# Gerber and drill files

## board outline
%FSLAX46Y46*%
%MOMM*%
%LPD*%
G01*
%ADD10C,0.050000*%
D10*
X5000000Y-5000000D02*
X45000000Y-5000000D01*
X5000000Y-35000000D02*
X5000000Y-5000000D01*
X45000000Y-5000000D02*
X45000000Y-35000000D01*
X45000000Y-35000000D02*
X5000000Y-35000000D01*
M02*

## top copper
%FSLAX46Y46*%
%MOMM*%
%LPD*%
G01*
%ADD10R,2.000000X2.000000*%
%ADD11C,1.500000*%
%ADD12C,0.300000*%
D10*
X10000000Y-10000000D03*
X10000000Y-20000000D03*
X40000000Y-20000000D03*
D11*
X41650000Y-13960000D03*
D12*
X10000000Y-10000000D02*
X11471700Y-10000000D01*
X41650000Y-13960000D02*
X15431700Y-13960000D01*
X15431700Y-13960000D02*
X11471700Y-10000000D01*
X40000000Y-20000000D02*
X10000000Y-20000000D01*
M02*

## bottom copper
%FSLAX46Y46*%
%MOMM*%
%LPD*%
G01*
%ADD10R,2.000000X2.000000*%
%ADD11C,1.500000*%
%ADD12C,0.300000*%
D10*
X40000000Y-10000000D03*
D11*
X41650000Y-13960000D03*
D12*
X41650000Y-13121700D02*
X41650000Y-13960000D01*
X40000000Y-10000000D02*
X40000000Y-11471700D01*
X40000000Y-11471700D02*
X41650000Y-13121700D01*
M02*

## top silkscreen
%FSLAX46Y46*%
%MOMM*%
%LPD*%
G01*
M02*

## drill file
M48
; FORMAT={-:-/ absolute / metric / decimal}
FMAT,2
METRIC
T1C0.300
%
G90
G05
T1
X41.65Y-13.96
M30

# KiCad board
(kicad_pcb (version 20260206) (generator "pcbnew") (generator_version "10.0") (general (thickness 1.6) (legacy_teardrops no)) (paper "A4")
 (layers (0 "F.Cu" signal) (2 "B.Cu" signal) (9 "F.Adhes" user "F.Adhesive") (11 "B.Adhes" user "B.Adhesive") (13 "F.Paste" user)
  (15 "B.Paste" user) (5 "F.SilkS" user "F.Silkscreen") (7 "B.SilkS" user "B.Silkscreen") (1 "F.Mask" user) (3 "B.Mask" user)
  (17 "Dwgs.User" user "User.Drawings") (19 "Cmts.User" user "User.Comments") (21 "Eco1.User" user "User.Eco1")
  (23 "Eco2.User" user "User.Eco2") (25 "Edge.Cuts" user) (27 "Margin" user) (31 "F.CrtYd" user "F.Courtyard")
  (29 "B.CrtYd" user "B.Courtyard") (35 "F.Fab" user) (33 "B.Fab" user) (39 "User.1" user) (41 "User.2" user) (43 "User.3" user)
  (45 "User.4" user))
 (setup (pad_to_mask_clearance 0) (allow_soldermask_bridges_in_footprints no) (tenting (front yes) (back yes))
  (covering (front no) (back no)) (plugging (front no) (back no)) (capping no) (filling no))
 (gr_line (start 5 5) (end 45 5) (stroke (width 0.05) (type default)) (layer "Edge.Cuts"))
 (gr_line (start 5 35) (end 5 5) (stroke (width 0.05) (type default)) (layer "Edge.Cuts"))
 (gr_line (start 45 5) (end 45 35) (stroke (width 0.05) (type default)) (layer "Edge.Cuts"))
 (gr_line (start 45 35) (end 5 35) (stroke (width 0.05) (type default)) (layer "Edge.Cuts"))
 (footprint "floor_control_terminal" (layer "F.Cu") (at 10 10)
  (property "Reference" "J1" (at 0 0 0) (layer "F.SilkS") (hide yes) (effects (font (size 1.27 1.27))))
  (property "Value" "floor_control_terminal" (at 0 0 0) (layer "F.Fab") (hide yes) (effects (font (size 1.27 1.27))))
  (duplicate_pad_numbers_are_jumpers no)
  (pad "1" smd rect (at 0 0) (size 2 2) (layers "F.Cu" "F.Paste" "F.Mask") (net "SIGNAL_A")))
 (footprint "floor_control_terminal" (layer "B.Cu") (at 40 10)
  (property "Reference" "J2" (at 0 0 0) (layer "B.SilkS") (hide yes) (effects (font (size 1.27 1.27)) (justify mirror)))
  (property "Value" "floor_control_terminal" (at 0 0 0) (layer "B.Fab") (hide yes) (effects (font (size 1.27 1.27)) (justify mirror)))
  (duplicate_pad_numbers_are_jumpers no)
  (pad "1" smd rect (at 0 0) (size 2 2) (layers "B.Cu" "B.Paste" "B.Mask") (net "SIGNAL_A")))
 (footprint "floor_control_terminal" (layer "F.Cu") (at 10 20)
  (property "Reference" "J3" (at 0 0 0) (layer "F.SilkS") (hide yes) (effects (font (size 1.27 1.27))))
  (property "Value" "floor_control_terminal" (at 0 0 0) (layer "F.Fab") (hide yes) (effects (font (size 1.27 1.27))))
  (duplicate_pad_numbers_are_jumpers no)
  (pad "1" smd rect (at 0 0) (size 2 2) (layers "F.Cu" "F.Paste" "F.Mask") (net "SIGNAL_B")))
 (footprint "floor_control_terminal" (layer "F.Cu") (at 40 20)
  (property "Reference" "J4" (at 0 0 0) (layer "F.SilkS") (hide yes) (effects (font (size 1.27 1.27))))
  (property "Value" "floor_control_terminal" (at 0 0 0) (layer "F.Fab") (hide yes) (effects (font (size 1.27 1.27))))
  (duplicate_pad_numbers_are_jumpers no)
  (pad "1" smd rect (at 0 0) (size 2 2) (layers "F.Cu" "F.Paste" "F.Mask") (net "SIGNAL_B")))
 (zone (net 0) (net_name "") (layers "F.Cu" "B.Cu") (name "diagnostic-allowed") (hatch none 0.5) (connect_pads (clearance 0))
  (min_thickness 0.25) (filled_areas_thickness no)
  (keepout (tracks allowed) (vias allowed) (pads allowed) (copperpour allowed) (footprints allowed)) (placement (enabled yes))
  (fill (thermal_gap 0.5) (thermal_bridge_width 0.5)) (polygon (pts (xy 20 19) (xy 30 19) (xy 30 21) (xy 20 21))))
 (segment (start 10 10) (end 11.4717 10) (width 0.3) (layer "F.Cu") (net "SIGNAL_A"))
 (segment (start 41.65 13.96) (end 15.4317 13.96) (width 0.3) (layer "F.Cu") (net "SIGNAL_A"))
 (segment (start 15.4317 13.96) (end 11.4717 10) (width 0.3) (layer "F.Cu") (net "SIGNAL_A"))
 (via (at 41.65 13.96) (size 1.5) (drill 0.3) (layers "F.Cu" "B.Cu") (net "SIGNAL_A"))
 (segment (start 41.65 13.1217) (end 41.65 13.96) (width 0.3) (layer "B.Cu") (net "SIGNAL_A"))
 (segment (start 40 10) (end 40 11.4717) (width 0.3) (layer "B.Cu") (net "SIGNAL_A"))
 (segment (start 40 11.4717) (end 41.65 13.1217) (width 0.3) (layer "B.Cu") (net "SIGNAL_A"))
 (segment (start 40 20) (end 10 20) (width 0.3) (layer "F.Cu") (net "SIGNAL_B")))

